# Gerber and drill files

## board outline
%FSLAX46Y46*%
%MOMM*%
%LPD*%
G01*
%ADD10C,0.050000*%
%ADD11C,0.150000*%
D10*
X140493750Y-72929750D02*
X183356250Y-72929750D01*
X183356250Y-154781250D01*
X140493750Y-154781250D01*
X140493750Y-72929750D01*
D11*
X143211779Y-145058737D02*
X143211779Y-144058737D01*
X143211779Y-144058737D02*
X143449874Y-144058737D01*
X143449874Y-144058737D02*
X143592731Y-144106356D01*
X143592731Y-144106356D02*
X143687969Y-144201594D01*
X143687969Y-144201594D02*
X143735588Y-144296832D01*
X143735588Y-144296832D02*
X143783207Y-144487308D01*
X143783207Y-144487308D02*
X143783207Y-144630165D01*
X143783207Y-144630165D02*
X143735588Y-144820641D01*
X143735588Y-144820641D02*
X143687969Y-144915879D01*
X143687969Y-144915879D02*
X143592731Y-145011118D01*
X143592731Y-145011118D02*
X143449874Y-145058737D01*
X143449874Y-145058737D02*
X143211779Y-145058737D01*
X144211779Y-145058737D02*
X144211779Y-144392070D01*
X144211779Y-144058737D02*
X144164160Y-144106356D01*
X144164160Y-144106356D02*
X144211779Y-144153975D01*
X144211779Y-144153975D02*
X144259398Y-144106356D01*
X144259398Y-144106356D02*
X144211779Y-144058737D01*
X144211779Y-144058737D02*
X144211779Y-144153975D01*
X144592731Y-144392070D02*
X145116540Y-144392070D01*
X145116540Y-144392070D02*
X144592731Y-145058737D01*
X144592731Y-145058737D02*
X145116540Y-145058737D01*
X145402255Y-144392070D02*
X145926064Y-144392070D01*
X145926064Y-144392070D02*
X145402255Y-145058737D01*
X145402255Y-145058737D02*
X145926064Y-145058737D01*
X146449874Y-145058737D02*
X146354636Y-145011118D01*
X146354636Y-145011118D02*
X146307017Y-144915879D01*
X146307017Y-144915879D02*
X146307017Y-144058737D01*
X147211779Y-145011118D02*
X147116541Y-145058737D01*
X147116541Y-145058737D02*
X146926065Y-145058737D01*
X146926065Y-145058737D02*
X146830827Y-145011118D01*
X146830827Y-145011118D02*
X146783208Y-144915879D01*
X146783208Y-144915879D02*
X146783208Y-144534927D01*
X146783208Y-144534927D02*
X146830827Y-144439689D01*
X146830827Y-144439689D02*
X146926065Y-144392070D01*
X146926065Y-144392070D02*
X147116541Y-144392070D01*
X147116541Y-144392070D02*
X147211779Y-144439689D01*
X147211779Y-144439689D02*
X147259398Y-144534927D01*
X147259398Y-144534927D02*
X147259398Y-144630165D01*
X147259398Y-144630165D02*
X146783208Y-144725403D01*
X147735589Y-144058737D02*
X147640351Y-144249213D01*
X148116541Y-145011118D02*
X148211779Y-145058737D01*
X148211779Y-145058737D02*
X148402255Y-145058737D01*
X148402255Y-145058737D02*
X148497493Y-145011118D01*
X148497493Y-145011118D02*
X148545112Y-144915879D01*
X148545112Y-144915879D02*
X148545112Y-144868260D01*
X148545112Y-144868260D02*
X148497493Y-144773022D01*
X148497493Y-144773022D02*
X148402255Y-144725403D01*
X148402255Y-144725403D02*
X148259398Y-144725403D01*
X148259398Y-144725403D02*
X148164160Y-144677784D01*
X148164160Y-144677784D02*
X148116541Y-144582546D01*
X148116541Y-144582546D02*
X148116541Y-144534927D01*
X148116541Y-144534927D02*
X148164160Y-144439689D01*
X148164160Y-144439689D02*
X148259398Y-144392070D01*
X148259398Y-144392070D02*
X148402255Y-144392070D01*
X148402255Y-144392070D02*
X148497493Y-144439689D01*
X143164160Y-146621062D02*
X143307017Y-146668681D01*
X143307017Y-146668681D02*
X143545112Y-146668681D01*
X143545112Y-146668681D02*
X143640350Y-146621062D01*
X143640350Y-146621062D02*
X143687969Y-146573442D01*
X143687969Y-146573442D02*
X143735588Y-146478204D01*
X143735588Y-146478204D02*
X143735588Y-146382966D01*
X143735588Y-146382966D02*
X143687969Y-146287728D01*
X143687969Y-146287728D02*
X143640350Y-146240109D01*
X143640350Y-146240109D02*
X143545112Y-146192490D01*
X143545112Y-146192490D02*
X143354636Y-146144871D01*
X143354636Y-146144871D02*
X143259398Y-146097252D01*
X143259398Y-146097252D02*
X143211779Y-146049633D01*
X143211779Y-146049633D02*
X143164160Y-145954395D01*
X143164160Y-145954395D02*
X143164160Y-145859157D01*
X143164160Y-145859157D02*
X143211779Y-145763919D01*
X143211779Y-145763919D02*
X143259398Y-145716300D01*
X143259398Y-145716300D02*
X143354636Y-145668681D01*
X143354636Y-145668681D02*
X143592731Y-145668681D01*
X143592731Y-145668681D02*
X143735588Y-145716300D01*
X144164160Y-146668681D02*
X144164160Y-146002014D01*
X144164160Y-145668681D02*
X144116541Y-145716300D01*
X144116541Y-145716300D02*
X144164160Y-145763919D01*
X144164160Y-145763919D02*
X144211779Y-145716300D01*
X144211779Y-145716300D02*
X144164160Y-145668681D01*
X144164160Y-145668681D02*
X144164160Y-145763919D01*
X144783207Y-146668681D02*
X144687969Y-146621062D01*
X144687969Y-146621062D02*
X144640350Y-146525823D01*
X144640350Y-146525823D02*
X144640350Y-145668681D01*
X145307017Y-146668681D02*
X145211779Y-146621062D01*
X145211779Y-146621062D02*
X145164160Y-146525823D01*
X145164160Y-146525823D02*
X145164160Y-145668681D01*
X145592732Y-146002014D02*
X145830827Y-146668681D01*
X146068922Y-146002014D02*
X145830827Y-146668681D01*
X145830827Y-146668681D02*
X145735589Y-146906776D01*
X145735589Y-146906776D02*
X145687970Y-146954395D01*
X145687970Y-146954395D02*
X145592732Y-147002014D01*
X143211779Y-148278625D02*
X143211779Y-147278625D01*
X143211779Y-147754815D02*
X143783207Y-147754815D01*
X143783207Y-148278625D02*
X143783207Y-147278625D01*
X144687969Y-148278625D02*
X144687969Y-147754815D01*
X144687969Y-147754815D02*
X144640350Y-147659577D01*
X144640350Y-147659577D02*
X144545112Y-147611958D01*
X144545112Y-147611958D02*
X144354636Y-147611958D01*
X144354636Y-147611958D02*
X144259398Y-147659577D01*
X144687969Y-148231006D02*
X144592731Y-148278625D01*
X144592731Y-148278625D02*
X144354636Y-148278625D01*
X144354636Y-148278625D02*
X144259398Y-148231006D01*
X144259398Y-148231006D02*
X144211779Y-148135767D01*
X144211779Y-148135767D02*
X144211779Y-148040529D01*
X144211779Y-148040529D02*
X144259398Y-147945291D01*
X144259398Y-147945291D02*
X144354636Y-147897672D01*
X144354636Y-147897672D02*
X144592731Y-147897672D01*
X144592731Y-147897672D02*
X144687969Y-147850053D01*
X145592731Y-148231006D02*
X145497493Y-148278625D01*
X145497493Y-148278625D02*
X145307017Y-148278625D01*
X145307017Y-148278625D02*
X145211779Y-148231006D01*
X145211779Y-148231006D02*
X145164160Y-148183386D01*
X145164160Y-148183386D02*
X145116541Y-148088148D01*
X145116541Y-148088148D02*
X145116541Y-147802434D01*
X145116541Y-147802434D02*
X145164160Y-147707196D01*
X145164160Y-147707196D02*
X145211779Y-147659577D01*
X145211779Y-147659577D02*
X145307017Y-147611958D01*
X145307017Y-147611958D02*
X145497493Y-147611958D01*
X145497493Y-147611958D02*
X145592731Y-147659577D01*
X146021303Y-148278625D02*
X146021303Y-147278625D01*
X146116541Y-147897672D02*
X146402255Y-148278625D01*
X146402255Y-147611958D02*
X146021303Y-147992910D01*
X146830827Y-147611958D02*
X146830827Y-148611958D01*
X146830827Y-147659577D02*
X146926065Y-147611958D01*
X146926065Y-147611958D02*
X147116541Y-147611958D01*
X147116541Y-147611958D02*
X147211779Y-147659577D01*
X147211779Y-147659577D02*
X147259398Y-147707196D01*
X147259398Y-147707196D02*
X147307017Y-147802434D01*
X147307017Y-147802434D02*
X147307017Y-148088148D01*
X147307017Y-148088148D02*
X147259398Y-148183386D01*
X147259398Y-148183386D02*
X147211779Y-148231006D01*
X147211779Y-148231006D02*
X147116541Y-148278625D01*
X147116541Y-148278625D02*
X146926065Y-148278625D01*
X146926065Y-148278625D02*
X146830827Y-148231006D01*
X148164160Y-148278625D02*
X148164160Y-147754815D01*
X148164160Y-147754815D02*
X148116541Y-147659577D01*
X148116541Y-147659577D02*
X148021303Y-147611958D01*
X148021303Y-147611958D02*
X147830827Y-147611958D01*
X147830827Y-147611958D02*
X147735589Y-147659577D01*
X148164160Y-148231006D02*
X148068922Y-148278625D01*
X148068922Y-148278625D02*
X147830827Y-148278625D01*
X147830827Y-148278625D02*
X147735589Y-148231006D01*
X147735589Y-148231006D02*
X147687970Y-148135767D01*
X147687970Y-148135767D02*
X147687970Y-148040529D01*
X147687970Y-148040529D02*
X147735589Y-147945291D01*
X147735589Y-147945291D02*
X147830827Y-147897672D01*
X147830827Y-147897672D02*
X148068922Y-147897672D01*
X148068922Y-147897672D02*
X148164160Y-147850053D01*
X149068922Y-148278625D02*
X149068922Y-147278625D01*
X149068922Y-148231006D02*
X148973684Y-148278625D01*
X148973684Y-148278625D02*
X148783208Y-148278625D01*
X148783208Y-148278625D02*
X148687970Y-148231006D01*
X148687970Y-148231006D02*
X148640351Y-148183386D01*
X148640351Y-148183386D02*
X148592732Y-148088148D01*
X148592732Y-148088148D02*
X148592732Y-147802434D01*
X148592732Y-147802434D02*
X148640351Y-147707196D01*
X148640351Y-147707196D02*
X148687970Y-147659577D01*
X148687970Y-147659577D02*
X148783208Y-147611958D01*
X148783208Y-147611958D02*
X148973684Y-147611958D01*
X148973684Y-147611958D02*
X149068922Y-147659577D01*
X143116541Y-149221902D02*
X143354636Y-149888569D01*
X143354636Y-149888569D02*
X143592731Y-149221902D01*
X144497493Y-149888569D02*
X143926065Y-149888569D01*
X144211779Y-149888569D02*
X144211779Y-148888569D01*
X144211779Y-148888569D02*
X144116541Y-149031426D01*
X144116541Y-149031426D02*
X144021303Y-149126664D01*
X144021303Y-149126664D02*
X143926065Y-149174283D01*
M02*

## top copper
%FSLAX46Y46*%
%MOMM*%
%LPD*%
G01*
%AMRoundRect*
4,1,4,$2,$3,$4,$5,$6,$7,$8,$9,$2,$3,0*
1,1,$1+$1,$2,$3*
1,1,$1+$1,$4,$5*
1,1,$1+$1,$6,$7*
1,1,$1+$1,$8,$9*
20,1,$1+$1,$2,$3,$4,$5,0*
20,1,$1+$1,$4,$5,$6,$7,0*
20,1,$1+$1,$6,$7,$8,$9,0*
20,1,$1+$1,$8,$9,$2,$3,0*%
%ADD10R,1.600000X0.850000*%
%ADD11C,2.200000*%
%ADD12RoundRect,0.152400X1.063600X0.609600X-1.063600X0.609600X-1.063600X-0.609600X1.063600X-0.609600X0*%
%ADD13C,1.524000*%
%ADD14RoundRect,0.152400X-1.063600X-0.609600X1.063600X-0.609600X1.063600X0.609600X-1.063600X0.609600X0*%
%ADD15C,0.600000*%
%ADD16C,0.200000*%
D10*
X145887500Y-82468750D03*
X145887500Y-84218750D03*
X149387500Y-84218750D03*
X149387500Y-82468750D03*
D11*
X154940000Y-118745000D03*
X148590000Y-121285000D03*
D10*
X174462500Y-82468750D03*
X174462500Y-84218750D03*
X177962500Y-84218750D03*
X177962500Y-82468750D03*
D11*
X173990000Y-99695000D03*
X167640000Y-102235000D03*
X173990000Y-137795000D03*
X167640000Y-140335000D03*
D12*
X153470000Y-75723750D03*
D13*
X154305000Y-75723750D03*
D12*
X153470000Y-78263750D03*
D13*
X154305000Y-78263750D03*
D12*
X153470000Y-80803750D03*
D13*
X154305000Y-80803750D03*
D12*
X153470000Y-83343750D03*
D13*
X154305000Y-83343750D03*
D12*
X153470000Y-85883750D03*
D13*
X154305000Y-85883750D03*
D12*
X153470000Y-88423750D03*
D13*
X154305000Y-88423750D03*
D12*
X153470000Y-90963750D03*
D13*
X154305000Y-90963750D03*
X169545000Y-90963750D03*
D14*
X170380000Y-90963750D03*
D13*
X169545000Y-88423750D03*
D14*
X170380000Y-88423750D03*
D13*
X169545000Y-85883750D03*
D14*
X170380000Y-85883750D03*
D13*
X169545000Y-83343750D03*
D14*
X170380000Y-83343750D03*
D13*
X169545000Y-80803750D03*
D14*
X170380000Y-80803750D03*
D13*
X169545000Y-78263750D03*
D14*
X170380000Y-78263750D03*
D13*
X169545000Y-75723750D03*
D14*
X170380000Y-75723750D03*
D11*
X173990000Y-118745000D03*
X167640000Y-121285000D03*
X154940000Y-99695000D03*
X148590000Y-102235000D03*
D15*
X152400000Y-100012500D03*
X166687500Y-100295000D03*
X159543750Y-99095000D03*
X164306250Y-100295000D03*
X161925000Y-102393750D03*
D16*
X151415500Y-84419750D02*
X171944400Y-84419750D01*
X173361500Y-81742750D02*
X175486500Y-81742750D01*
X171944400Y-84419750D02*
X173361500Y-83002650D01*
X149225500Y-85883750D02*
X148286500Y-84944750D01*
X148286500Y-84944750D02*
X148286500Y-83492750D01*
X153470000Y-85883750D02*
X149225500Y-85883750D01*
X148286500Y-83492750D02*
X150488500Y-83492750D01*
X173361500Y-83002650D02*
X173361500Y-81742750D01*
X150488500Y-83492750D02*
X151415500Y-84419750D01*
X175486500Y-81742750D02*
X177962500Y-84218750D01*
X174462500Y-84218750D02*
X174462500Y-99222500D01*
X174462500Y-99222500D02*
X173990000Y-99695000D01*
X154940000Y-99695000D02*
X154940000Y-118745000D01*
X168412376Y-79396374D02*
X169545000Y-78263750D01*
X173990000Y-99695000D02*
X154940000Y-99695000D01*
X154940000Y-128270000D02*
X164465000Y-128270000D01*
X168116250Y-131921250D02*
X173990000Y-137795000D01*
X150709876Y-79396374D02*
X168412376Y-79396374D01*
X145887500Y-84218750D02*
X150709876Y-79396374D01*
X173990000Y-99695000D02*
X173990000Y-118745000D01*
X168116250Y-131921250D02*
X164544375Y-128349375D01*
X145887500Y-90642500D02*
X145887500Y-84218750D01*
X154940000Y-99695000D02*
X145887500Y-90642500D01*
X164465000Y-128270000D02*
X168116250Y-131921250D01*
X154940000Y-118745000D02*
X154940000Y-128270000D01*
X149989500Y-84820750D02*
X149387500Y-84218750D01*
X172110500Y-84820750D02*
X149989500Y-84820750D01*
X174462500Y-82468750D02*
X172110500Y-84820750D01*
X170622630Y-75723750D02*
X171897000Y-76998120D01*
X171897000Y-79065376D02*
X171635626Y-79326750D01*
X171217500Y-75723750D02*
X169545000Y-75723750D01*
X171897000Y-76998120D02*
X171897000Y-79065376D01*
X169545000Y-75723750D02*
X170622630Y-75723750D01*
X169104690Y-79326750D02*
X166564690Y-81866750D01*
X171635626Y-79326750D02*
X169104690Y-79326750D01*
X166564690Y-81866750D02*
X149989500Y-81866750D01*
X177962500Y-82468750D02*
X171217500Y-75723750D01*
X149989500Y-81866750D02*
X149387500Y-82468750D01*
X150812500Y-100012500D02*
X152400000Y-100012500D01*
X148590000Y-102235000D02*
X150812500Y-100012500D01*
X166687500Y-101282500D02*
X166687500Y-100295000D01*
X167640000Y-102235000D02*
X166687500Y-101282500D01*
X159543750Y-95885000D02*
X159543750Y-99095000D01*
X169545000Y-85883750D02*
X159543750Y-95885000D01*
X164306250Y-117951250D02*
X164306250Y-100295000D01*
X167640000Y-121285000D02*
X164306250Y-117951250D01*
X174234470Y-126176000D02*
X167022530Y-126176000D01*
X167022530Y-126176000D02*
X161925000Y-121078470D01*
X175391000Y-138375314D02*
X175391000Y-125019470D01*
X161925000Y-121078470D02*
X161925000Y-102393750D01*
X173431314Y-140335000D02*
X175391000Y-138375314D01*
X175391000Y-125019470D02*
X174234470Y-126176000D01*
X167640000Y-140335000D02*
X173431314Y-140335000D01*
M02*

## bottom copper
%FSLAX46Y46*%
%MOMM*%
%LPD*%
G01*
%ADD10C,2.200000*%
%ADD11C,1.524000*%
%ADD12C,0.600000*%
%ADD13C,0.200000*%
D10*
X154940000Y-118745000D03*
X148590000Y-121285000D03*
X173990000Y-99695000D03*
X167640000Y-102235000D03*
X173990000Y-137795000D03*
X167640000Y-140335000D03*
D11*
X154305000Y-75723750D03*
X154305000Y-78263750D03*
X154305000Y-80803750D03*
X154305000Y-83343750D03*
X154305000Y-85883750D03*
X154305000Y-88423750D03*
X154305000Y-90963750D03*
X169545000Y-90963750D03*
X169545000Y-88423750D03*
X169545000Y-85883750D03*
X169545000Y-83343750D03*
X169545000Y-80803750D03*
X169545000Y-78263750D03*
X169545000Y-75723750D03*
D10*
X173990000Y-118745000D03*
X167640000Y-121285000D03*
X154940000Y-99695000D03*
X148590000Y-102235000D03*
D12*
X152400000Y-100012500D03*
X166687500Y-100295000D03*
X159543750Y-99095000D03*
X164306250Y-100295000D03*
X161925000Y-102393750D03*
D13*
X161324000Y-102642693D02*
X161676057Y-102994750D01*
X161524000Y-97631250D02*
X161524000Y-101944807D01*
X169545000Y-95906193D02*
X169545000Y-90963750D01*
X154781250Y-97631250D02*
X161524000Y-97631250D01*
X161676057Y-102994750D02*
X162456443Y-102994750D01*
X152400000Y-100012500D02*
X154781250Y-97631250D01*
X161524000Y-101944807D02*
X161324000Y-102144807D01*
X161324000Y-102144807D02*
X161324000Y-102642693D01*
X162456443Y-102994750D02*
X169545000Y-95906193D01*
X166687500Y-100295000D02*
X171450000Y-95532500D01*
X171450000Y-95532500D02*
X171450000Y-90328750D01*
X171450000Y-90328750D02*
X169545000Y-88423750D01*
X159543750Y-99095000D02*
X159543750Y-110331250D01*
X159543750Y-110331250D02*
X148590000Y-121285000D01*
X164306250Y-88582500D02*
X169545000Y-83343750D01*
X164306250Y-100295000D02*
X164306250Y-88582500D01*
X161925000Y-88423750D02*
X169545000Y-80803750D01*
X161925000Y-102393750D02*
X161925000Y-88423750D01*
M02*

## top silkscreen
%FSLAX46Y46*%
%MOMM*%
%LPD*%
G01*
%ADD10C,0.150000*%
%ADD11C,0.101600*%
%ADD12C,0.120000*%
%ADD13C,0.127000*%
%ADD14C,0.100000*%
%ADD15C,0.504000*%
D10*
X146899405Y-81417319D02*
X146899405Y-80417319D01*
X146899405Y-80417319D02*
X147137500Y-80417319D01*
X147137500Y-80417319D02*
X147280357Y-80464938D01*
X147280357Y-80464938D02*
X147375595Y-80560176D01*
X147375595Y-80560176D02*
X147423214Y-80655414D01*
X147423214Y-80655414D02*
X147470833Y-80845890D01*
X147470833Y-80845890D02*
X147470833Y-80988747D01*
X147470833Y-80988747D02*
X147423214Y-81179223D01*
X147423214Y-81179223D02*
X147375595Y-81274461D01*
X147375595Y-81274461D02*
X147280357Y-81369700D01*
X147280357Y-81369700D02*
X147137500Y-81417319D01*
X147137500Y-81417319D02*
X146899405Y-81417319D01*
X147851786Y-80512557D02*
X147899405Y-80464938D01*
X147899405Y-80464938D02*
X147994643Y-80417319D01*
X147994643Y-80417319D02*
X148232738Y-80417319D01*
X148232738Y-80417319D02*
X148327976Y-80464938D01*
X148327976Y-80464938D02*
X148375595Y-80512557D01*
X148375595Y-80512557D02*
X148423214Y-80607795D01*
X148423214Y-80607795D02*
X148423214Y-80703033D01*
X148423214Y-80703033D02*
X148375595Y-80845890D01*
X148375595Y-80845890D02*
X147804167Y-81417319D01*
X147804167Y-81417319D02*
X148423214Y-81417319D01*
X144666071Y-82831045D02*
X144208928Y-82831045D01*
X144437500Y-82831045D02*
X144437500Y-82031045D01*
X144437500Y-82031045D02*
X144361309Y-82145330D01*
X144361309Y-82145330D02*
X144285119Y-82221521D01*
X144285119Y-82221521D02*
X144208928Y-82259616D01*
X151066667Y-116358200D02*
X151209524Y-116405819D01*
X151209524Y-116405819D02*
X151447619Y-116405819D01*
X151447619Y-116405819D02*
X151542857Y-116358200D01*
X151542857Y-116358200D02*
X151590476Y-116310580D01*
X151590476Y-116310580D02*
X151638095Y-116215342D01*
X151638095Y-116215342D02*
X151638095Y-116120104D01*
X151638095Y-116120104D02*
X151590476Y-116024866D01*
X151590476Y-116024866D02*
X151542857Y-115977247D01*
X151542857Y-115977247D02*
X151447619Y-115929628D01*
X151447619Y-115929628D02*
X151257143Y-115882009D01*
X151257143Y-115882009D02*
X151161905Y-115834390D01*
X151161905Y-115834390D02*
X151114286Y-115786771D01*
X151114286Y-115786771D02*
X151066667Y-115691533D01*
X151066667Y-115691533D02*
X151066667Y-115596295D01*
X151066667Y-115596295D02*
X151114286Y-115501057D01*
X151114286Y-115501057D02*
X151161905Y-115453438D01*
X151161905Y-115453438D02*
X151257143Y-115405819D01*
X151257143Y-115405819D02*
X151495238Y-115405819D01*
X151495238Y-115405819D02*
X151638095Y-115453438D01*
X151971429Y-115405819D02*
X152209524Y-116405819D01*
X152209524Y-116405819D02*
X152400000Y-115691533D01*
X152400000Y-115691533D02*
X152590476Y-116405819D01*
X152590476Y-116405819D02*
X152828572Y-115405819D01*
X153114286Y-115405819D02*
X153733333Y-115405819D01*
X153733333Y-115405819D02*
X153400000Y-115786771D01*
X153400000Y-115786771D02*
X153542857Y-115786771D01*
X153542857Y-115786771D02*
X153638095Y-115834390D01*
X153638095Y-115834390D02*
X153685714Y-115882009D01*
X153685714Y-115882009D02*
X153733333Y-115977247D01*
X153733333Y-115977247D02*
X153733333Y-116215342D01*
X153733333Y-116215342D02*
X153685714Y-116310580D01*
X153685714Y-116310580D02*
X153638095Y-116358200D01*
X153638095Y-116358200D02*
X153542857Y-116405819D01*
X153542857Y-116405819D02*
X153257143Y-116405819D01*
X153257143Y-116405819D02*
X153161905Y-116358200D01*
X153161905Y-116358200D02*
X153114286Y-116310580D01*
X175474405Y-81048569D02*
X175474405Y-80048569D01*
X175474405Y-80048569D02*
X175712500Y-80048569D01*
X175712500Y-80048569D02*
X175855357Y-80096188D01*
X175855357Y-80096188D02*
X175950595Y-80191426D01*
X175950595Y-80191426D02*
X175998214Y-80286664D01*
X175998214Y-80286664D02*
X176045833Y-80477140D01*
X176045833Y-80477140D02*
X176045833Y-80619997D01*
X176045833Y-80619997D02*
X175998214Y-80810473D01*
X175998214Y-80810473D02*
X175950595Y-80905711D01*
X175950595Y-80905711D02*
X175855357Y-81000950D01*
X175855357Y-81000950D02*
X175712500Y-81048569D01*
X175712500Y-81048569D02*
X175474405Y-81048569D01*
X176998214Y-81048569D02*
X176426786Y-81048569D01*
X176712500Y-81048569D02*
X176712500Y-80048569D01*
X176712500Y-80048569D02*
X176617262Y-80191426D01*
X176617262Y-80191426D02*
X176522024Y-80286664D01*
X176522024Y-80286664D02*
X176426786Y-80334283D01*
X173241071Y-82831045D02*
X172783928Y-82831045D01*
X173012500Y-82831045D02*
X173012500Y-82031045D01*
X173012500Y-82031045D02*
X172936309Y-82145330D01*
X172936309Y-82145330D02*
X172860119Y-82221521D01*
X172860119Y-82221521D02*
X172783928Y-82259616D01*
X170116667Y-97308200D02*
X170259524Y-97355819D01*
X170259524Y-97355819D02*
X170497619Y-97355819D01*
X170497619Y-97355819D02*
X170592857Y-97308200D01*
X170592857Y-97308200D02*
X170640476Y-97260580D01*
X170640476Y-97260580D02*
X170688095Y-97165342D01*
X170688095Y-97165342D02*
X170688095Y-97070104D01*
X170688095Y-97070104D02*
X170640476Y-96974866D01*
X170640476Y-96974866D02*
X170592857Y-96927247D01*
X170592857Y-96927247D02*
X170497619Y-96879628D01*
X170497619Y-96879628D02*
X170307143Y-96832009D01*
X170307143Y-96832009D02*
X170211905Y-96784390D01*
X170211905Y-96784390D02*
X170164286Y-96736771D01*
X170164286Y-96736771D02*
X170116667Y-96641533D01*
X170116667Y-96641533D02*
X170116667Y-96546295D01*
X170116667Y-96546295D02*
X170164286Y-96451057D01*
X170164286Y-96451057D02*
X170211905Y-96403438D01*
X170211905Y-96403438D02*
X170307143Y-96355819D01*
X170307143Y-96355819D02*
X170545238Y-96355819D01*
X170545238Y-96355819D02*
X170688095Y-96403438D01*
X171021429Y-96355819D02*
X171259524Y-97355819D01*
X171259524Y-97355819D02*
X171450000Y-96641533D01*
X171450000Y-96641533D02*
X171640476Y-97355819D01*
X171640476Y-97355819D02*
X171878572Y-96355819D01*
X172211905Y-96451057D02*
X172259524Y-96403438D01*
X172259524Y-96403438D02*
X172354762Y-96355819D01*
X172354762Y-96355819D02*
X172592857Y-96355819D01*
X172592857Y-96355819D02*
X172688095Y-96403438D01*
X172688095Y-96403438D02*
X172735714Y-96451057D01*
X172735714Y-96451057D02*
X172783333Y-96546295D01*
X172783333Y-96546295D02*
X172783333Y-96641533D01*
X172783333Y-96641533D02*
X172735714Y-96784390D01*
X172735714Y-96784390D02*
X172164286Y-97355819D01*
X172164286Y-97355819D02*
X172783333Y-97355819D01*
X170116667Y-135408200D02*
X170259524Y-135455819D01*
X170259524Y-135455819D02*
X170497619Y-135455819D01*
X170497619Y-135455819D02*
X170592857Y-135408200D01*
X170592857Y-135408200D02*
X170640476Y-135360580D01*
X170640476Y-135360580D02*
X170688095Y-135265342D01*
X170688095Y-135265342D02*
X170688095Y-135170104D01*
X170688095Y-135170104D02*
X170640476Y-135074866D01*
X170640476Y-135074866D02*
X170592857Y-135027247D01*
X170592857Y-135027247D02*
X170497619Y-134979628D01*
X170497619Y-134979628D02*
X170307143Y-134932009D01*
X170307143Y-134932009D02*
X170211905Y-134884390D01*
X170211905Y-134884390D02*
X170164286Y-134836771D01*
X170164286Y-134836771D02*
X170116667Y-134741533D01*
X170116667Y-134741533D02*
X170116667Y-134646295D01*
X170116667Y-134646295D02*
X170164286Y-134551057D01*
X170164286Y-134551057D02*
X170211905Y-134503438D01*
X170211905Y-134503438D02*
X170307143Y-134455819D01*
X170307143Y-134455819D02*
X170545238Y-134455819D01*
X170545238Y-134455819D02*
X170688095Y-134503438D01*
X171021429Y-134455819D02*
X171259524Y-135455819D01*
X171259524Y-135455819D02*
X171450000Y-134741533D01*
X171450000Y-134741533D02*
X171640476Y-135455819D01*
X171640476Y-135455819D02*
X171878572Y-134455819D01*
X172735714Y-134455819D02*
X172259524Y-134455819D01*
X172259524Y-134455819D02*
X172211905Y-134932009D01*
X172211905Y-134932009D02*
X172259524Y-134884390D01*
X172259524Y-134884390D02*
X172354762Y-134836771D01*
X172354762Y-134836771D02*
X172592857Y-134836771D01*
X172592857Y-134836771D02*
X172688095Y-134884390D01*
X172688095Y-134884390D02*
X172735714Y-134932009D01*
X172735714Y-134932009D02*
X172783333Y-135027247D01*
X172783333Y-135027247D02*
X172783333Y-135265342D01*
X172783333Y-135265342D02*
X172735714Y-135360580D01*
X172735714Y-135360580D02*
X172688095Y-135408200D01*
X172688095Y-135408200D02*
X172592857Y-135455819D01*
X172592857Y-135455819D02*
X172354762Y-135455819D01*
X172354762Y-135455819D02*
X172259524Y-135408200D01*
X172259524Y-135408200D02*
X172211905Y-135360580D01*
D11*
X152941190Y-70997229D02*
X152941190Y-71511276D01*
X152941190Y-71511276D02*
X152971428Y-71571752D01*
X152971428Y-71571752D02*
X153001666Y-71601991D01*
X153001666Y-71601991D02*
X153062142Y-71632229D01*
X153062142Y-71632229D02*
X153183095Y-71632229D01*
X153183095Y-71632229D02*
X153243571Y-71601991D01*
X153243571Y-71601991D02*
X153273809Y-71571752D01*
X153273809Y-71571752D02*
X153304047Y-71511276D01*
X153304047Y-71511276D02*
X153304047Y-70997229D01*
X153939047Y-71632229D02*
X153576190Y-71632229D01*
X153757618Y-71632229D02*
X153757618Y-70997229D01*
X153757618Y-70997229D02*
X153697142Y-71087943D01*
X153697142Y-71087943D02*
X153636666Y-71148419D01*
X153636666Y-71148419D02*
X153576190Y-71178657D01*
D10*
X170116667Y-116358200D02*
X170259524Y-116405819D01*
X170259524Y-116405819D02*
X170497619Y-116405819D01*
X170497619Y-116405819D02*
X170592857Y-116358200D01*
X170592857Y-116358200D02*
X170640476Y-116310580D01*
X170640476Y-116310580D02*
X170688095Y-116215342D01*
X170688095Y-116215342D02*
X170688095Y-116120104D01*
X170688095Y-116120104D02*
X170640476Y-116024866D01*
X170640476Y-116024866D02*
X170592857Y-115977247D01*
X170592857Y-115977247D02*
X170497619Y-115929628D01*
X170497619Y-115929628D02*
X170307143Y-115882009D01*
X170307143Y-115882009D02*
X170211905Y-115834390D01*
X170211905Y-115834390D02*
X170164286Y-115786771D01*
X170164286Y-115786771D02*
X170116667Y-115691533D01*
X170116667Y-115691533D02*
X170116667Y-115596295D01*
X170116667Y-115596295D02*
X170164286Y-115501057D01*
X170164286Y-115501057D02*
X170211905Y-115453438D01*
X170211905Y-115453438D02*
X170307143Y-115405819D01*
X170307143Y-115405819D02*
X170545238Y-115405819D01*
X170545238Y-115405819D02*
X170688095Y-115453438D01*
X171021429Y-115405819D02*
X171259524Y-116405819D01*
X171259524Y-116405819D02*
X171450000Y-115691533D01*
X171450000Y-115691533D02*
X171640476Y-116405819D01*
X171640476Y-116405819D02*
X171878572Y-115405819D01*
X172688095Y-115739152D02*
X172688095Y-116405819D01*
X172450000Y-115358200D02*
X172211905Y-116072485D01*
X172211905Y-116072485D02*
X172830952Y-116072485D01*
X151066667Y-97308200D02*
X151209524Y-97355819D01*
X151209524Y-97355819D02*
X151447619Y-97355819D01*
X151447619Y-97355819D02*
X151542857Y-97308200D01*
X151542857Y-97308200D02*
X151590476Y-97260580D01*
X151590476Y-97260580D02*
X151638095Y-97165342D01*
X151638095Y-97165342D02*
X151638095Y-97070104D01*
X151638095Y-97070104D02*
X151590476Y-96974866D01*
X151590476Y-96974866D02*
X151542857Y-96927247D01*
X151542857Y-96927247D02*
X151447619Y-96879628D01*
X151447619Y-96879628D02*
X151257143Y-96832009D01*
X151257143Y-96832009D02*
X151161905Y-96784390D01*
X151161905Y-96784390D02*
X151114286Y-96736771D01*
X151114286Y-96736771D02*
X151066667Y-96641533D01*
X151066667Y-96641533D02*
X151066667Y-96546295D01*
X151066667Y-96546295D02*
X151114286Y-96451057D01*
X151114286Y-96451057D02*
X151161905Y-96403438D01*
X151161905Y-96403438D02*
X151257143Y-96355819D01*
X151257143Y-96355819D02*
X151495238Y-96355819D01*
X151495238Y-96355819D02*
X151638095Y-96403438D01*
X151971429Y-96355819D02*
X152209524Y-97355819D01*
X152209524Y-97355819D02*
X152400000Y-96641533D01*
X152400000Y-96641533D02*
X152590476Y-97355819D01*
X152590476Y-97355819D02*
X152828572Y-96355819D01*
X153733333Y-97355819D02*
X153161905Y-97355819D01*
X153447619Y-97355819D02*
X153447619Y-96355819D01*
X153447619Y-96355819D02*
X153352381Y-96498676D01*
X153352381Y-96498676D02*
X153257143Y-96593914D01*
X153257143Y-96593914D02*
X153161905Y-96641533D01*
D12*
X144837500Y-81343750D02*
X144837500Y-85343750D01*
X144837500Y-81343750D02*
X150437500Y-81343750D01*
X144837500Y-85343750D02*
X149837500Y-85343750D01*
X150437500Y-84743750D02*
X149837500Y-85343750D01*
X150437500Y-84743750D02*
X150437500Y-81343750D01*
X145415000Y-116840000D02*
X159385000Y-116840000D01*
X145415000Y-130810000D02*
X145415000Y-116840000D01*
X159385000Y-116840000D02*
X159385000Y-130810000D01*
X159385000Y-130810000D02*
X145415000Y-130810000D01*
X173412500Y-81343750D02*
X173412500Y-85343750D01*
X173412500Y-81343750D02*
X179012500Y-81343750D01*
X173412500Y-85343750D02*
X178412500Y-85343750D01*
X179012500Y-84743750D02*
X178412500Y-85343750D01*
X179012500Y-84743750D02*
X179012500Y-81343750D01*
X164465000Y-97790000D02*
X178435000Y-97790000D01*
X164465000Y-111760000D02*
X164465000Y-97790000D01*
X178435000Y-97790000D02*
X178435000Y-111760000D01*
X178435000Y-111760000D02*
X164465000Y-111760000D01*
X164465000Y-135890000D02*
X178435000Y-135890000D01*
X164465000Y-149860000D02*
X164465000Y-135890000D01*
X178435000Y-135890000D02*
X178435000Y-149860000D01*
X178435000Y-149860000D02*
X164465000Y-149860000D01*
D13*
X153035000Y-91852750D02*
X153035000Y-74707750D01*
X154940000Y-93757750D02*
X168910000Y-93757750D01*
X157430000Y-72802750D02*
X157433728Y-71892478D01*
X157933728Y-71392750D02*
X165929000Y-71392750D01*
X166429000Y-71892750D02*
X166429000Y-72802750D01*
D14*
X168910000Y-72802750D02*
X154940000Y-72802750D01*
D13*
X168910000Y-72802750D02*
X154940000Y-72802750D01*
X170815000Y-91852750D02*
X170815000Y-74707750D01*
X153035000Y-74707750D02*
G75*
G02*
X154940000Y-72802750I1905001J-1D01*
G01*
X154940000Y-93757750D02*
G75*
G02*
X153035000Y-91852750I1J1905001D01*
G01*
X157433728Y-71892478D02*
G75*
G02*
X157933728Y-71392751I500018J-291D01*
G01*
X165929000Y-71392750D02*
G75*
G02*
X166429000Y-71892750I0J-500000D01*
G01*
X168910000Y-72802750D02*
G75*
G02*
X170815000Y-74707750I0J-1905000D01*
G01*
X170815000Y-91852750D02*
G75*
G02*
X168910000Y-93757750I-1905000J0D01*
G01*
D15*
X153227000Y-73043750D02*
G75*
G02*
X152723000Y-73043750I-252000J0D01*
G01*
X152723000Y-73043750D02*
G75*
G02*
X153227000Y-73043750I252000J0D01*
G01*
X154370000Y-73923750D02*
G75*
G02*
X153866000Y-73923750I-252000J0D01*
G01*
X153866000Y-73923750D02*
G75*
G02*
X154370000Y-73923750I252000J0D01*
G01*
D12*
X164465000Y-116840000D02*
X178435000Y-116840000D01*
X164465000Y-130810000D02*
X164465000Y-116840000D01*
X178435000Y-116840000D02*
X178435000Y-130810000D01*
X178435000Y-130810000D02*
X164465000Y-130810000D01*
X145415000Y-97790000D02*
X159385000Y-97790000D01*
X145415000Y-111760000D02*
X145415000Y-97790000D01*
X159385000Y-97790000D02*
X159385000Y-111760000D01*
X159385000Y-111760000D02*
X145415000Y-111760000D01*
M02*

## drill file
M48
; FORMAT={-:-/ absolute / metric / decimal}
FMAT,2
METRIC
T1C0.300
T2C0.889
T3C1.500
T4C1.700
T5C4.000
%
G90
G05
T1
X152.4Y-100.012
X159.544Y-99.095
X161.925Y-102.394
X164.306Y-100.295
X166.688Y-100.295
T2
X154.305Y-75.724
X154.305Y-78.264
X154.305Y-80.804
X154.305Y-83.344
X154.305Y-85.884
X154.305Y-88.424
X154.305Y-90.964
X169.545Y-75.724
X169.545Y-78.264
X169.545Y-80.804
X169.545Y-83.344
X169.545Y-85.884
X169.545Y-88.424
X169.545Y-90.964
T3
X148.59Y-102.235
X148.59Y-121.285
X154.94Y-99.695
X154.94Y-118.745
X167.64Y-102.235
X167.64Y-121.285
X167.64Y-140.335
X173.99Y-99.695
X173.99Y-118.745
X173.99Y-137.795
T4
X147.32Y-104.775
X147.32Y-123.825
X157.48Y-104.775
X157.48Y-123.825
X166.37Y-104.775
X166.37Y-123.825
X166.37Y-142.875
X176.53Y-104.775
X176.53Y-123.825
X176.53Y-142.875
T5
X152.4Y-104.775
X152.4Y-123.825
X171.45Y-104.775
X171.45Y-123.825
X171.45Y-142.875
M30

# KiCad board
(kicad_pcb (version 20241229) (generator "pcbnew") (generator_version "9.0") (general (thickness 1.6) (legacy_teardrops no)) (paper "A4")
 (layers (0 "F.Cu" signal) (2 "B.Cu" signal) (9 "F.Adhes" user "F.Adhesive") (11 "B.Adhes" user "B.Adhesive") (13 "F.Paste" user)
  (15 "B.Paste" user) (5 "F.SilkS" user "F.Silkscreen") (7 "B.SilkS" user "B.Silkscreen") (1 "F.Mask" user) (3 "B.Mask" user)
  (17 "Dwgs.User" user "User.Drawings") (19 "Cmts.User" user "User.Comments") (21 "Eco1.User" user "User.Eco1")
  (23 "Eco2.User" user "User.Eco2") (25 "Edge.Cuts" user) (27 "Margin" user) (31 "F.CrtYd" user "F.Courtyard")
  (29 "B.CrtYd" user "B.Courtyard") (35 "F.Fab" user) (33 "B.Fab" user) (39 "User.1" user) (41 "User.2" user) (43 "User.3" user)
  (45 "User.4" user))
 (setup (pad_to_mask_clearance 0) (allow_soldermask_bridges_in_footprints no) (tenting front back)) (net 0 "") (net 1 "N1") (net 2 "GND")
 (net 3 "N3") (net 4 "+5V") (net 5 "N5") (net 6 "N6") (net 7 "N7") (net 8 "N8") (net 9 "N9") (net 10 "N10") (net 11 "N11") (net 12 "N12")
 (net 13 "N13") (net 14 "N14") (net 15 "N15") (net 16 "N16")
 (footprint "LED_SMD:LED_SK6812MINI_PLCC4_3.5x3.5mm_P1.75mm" (layer "F.Cu") (at 147.6375 83.34375)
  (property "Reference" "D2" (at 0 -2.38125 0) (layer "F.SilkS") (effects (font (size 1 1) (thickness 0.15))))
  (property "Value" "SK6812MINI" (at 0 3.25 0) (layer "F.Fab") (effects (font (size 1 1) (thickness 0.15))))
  (fp_line (start -2.8 -2) (end -2.8 2) (stroke (width 0.12) (type default)) (layer "F.SilkS"))
  (fp_line (start -2.8 -2) (end 2.8 -2) (stroke (width 0.12) (type solid)) (layer "F.SilkS"))
  (fp_line (start -2.8 2) (end 2.2 2) (stroke (width 0.12) (type solid)) (layer "F.SilkS"))
  (fp_line (start 2.8 1.4) (end 2.2 2) (stroke (width 0.12) (type default)) (layer "F.SilkS"))
  (fp_line (start 2.8 1.4) (end 2.8 -2) (stroke (width 0.12) (type solid)) (layer "F.SilkS"))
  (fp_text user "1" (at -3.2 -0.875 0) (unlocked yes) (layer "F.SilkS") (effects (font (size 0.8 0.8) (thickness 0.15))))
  (pad "1" smd rect (at -1.75 -0.875) (size 1.6 0.85) (layers "F.Cu" "F.Mask" "F.Paste") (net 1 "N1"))
  (pad "2" smd rect (at -1.75 0.875) (size 1.6 0.85) (layers "F.Cu" "F.Mask" "F.Paste") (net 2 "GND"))
  (pad "3" smd rect (at 1.75 0.875) (size 1.6 0.85) (layers "F.Cu" "F.Mask" "F.Paste") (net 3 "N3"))
  (pad "4" smd rect (at 1.75 -0.875) (size 1.6 0.85) (layers "F.Cu" "F.Mask" "F.Paste") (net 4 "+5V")))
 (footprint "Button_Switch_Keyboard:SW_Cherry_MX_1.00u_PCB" (layer "F.Cu") (at 154.94 118.745)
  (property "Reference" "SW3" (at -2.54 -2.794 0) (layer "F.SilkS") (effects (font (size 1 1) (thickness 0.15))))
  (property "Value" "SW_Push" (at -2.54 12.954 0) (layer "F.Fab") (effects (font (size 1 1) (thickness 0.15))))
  (fp_line (start -9.525 -1.905) (end 4.445 -1.905) (stroke (width 0.12) (type solid)) (layer "F.SilkS"))
  (fp_line (start -9.525 12.065) (end -9.525 -1.905) (stroke (width 0.12) (type solid)) (layer "F.SilkS"))
  (fp_line (start 4.445 -1.905) (end 4.445 12.065) (stroke (width 0.12) (type solid)) (layer "F.SilkS"))
  (fp_line (start 4.445 12.065) (end -9.525 12.065) (stroke (width 0.12) (type solid)) (layer "F.SilkS"))
  (pad "" np_thru_hole circle (at -7.62 5.08) (size 1.7 1.7) (drill 1.7) (layers "*.Cu" "*.Mask"))
  (pad "" np_thru_hole circle (at -2.54 5.08) (size 4 4) (drill 4) (layers "*.Cu" "*.Mask"))
  (pad "" np_thru_hole circle (at 2.54 5.08) (size 1.7 1.7) (drill 1.7) (layers "*.Cu" "*.Mask"))
  (pad "1" thru_hole circle (at 0 0) (size 2.2 2.2) (drill 1.5) (layers "*.Cu" "*.Mask") (remove_unused_layers no) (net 2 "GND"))
  (pad "2" thru_hole circle (at -6.35 2.54) (size 2.2 2.2) (drill 1.5) (layers "*.Cu" "*.Mask") (remove_unused_layers no) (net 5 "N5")))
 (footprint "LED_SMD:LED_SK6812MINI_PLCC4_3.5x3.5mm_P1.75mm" (layer "F.Cu") (at 176.2125 83.34375)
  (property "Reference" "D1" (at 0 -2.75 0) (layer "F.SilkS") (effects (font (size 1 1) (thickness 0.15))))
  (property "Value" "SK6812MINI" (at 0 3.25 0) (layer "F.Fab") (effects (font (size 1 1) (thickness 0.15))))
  (fp_line (start -2.8 -2) (end -2.8 2) (stroke (width 0.12) (type default)) (layer "F.SilkS"))
  (fp_line (start -2.8 -2) (end 2.8 -2) (stroke (width 0.12) (type solid)) (layer "F.SilkS"))
  (fp_line (start -2.8 2) (end 2.2 2) (stroke (width 0.12) (type solid)) (layer "F.SilkS"))
  (fp_line (start 2.8 1.4) (end 2.2 2) (stroke (width 0.12) (type default)) (layer "F.SilkS"))
  (fp_line (start 2.8 1.4) (end 2.8 -2) (stroke (width 0.12) (type solid)) (layer "F.SilkS"))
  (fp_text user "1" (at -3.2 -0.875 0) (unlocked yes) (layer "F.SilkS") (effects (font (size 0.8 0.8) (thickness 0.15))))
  (pad "1" smd rect (at -1.75 -0.875) (size 1.6 0.85) (layers "F.Cu" "F.Mask" "F.Paste") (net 3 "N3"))
  (pad "2" smd rect (at -1.75 0.875) (size 1.6 0.85) (layers "F.Cu" "F.Mask" "F.Paste") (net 2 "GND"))
  (pad "3" smd rect (at 1.75 0.875) (size 1.6 0.85) (layers "F.Cu" "F.Mask" "F.Paste") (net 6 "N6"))
  (pad "4" smd rect (at 1.75 -0.875) (size 1.6 0.85) (layers "F.Cu" "F.Mask" "F.Paste") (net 4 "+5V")))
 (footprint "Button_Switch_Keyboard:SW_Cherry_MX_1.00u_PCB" (layer "F.Cu") (at 173.99 99.695)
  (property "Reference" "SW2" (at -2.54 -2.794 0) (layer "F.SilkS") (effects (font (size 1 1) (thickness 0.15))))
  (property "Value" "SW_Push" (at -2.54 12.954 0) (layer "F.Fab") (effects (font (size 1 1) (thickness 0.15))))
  (fp_line (start -9.525 -1.905) (end 4.445 -1.905) (stroke (width 0.12) (type solid)) (layer "F.SilkS"))
  (fp_line (start -9.525 12.065) (end -9.525 -1.905) (stroke (width 0.12) (type solid)) (layer "F.SilkS"))
  (fp_line (start 4.445 -1.905) (end 4.445 12.065) (stroke (width 0.12) (type solid)) (layer "F.SilkS"))
  (fp_line (start 4.445 12.065) (end -9.525 12.065) (stroke (width 0.12) (type solid)) (layer "F.SilkS"))
  (pad "" np_thru_hole circle (at -7.62 5.08) (size 1.7 1.7) (drill 1.7) (layers "*.Cu" "*.Mask"))
  (pad "" np_thru_hole circle (at -2.54 5.08) (size 4 4) (drill 4) (layers "*.Cu" "*.Mask"))
  (pad "" np_thru_hole circle (at 2.54 5.08) (size 1.7 1.7) (drill 1.7) (layers "*.Cu" "*.Mask"))
  (pad "1" thru_hole circle (at 0 0) (size 2.2 2.2) (drill 1.5) (layers "*.Cu" "*.Mask") (remove_unused_layers no) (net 2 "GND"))
  (pad "2" thru_hole circle (at -6.35 2.54) (size 2.2 2.2) (drill 1.5) (layers "*.Cu" "*.Mask") (remove_unused_layers no) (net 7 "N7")))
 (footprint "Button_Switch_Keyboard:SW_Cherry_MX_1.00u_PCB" (layer "F.Cu") (at 173.99 137.795)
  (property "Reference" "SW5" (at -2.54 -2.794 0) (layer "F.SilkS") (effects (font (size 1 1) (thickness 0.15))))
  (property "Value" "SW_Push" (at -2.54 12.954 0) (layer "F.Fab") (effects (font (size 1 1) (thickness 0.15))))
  (fp_line (start -9.525 -1.905) (end 4.445 -1.905) (stroke (width 0.12) (type solid)) (layer "F.SilkS"))
  (fp_line (start -9.525 12.065) (end -9.525 -1.905) (stroke (width 0.12) (type solid)) (layer "F.SilkS"))
  (fp_line (start 4.445 -1.905) (end 4.445 12.065) (stroke (width 0.12) (type solid)) (layer "F.SilkS"))
  (fp_line (start 4.445 12.065) (end -9.525 12.065) (stroke (width 0.12) (type solid)) (layer "F.SilkS"))
  (pad "" np_thru_hole circle (at -7.62 5.08) (size 1.7 1.7) (drill 1.7) (layers "*.Cu" "*.Mask"))
  (pad "" np_thru_hole circle (at -2.54 5.08) (size 4 4) (drill 4) (layers "*.Cu" "*.Mask"))
  (pad "" np_thru_hole circle (at 2.54 5.08) (size 1.7 1.7) (drill 1.7) (layers "*.Cu" "*.Mask"))
  (pad "1" thru_hole circle (at 0 0) (size 2.2 2.2) (drill 1.5) (layers "*.Cu" "*.Mask") (remove_unused_layers no) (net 2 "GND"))
  (pad "2" thru_hole circle (at -6.35 2.54) (size 2.2 2.2) (drill 1.5) (layers "*.Cu" "*.Mask") (remove_unused_layers no) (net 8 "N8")))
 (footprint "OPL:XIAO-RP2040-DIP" (layer "F.Cu") (at 161.925 83.34375)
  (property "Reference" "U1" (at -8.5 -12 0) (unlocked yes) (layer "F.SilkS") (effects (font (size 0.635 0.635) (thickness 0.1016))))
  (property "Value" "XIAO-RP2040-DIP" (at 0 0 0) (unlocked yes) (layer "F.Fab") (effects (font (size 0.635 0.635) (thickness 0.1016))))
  (fp_line (start -8.89 8.509) (end -8.89 -8.636) (stroke (width 0.127) (type solid)) (layer "F.SilkS"))
  (fp_line (start -6.985 10.414) (end 6.985 10.414) (stroke (width 0.127) (type solid)) (layer "F.SilkS"))
  (fp_line (start -4.495 -10.541) (end -4.491272 -11.451272) (stroke (width 0.127) (type solid)) (layer "F.SilkS"))
  (fp_line (start -3.991272 -11.951) (end 4.004 -11.951) (stroke (width 0.127) (type solid)) (layer "F.SilkS"))
  (fp_line (start 4.504 -11.451) (end 4.504 -10.541) (stroke (width 0.127) (type solid)) (layer "F.SilkS"))
  (fp_line (start 6.985 -10.541) (end -6.985 -10.541) (stroke (width 0.1) (type solid)) (layer "F.SilkS"))
  (fp_line (start 6.985 -10.541) (end -6.985 -10.541) (stroke (width 0.127) (type solid)) (layer "F.SilkS"))
  (fp_line (start 8.89 8.509) (end 8.89 -8.636) (stroke (width 0.127) (type solid)) (layer "F.SilkS"))
  (fp_arc (start -8.89 -8.636) (mid -8.332038 -9.983038) (end -6.985 -10.541) (stroke (width 0.127) (type solid)) (layer "F.SilkS"))
  (fp_arc (start -6.985 10.414) (mid -8.332038 9.856038) (end -8.89 8.509) (stroke (width 0.127) (type solid)) (layer "F.SilkS"))
  (fp_arc (start -4.491272 -11.451272) (mid -4.344728 -11.80464) (end -3.991272 -11.951) (stroke (width 0.127) (type default))
   (layer "F.SilkS"))
  (fp_arc (start 4.004 -11.951) (mid 4.357553 -11.804553) (end 4.504 -11.451) (stroke (width 0.127) (type default)) (layer "F.SilkS"))
  (fp_arc (start 6.985 -10.541) (mid 8.332038 -9.983038) (end 8.89 -8.636) (stroke (width 0.127) (type solid)) (layer "F.SilkS"))
  (fp_arc (start 8.89 8.509) (mid 8.332038 9.856038) (end 6.985 10.414) (stroke (width 0.127) (type solid)) (layer "F.SilkS"))
  (fp_circle (center -8.95 -10.3) (end -8.95 -10.554) (stroke (width 0.5) (type solid)) (fill yes) (layer "F.SilkS"))
  (fp_circle (center -7.807 -9.42) (end -7.807 -9.674) (stroke (width 0.5) (type solid)) (fill yes) (layer "F.SilkS"))
  (pad "1" smd roundrect (at -8.455 -7.62 180) (size 2.432 1.524) (layers "F.Cu" "F.Mask") (roundrect_rratio 0.1) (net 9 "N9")
   (thermal_bridge_angle 45))
  (pad "1" thru_hole circle (at -7.62 -7.62 180) (size 1.524 1.524) (drill 0.889) (layers "*.Cu" "*.Mask") (remove_unused_layers no)
   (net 9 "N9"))
  (pad "2" smd roundrect (at -8.455 -5.08 180) (size 2.432 1.524) (layers "F.Cu" "F.Mask") (roundrect_rratio 0.1) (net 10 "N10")
   (thermal_bridge_angle 45))
  (pad "2" thru_hole circle (at -7.62 -5.08 180) (size 1.524 1.524) (drill 0.889) (layers "*.Cu" "*.Mask") (remove_unused_layers no)
   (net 10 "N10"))
  (pad "3" smd roundrect (at -8.455 -2.54 180) (size 2.432 1.524) (layers "F.Cu" "F.Mask") (roundrect_rratio 0.1) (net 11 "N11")
   (thermal_bridge_angle 45))
  (pad "3" thru_hole circle (at -7.62 -2.54 180) (size 1.524 1.524) (drill 0.889) (layers "*.Cu" "*.Mask") (remove_unused_layers no)
   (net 11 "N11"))
  (pad "4" smd roundrect (at -8.455 0 180) (size 2.432 1.524) (layers "F.Cu" "F.Mask") (roundrect_rratio 0.1) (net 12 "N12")
   (thermal_bridge_angle 45))
  (pad "4" thru_hole circle (at -7.62 0 180) (size 1.524 1.524) (drill 0.889) (layers "*.Cu" "*.Mask") (remove_unused_layers no)
   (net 12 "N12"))
  (pad "5" smd roundrect (at -8.455 2.54 180) (size 2.432 1.524) (layers "F.Cu" "F.Mask") (roundrect_rratio 0.1) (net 6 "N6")
   (thermal_bridge_angle 45))
  (pad "5" thru_hole circle (at -7.62 2.54 180) (size 1.524 1.524) (drill 0.889) (layers "*.Cu" "*.Mask") (remove_unused_layers no)
   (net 6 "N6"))
  (pad "6" smd roundrect (at -8.455 5.08 180) (size 2.432 1.524) (layers "F.Cu" "F.Mask") (roundrect_rratio 0.1) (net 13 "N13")
   (thermal_bridge_angle 45))
  (pad "6" thru_hole circle (at -7.62 5.08 180) (size 1.524 1.524) (drill 0.889) (layers "*.Cu" "*.Mask") (remove_unused_layers no)
   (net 13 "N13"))
  (pad "7" smd roundrect (at -8.455 7.62 180) (size 2.432 1.524) (layers "F.Cu" "F.Mask") (roundrect_rratio 0.1) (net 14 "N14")
   (thermal_bridge_angle 45))
  (pad "7" thru_hole circle (at -7.62 7.62 180) (size 1.524 1.524) (drill 0.889) (layers "*.Cu" "*.Mask") (remove_unused_layers no)
   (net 14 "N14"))
  (pad "8" thru_hole circle (at 7.62 7.62) (size 1.524 1.524) (drill 0.889) (layers "*.Cu" "*.Mask") (remove_unused_layers no)
   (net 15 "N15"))
  (pad "8" smd roundrect (at 8.455 7.62) (size 2.432 1.524) (layers "F.Cu" "F.Mask") (roundrect_rratio 0.1) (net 15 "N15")
   (thermal_bridge_angle 45))
  (pad "9" thru_hole circle (at 7.62 5.08) (size 1.524 1.524) (drill 0.889) (layers "*.Cu" "*.Mask") (remove_unused_layers no) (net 7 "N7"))
  (pad "9" smd roundrect (at 8.455 5.08) (size 2.432 1.524) (layers "F.Cu" "F.Mask") (roundrect_rratio 0.1) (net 7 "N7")
   (thermal_bridge_angle 45))
  (pad "10" thru_hole circle (at 7.62 2.54) (size 1.524 1.524) (drill 0.889) (layers "*.Cu" "*.Mask") (remove_unused_layers no) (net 5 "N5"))
  (pad "10" smd roundrect (at 8.455 2.54) (size 2.432 1.524) (layers "F.Cu" "F.Mask") (roundrect_rratio 0.1) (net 5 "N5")
   (thermal_bridge_angle 45))
  (pad "11" thru_hole circle (at 7.62 0) (size 1.524 1.524) (drill 0.889) (layers "*.Cu" "*.Mask") (remove_unused_layers no) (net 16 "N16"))
  (pad "11" smd roundrect (at 8.455 0) (size 2.432 1.524) (layers "F.Cu" "F.Mask") (roundrect_rratio 0.1) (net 16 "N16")
   (thermal_bridge_angle 45))
  (pad "12" thru_hole circle (at 7.62 -2.54) (size 1.524 1.524) (drill 0.889) (layers "*.Cu" "*.Mask") (remove_unused_layers no)
   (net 8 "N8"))
  (pad "12" smd roundrect (at 8.455 -2.54) (size 2.432 1.524) (layers "F.Cu" "F.Mask") (roundrect_rratio 0.1) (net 8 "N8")
   (thermal_bridge_angle 45))
  (pad "13" thru_hole circle (at 7.62 -5.08) (size 1.524 1.524) (drill 0.889) (layers "*.Cu" "*.Mask") (remove_unused_layers no)
   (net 2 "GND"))
  (pad "13" smd roundrect (at 8.455 -5.08) (size 2.432 1.524) (layers "F.Cu" "F.Mask") (roundrect_rratio 0.1) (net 2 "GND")
   (thermal_bridge_angle 45))
  (pad "14" thru_hole circle (at 7.62 -7.62) (size 1.524 1.524) (drill 0.889) (layers "*.Cu" "*.Mask") (remove_unused_layers no)
   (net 4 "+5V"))
  (pad "14" smd roundrect (at 8.455 -7.62) (size 2.432 1.524) (layers "F.Cu" "F.Mask") (roundrect_rratio 0.1) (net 4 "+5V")
   (thermal_bridge_angle 45)))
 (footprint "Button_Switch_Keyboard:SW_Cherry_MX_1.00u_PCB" (layer "F.Cu") (at 173.99 118.745)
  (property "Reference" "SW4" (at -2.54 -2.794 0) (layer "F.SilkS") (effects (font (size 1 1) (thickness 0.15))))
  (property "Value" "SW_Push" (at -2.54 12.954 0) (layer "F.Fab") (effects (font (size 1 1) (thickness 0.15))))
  (fp_line (start -9.525 -1.905) (end 4.445 -1.905) (stroke (width 0.12) (type solid)) (layer "F.SilkS"))
  (fp_line (start -9.525 12.065) (end -9.525 -1.905) (stroke (width 0.12) (type solid)) (layer "F.SilkS"))
  (fp_line (start 4.445 -1.905) (end 4.445 12.065) (stroke (width 0.12) (type solid)) (layer "F.SilkS"))
  (fp_line (start 4.445 12.065) (end -9.525 12.065) (stroke (width 0.12) (type solid)) (layer "F.SilkS"))
  (pad "" np_thru_hole circle (at -7.62 5.08) (size 1.7 1.7) (drill 1.7) (layers "*.Cu" "*.Mask"))
  (pad "" np_thru_hole circle (at -2.54 5.08) (size 4 4) (drill 4) (layers "*.Cu" "*.Mask"))
  (pad "" np_thru_hole circle (at 2.54 5.08) (size 1.7 1.7) (drill 1.7) (layers "*.Cu" "*.Mask"))
  (pad "1" thru_hole circle (at 0 0) (size 2.2 2.2) (drill 1.5) (layers "*.Cu" "*.Mask") (remove_unused_layers no) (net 2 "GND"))
  (pad "2" thru_hole circle (at -6.35 2.54) (size 2.2 2.2) (drill 1.5) (layers "*.Cu" "*.Mask") (remove_unused_layers no) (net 16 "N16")))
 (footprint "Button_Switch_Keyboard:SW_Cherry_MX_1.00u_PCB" (layer "F.Cu") (at 154.94 99.695)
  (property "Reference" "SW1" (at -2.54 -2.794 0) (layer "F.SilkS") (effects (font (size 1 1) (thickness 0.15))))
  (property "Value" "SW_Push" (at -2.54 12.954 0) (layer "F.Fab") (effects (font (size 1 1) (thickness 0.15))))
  (fp_line (start -9.525 -1.905) (end 4.445 -1.905) (stroke (width 0.12) (type solid)) (layer "F.SilkS"))
  (fp_line (start -9.525 12.065) (end -9.525 -1.905) (stroke (width 0.12) (type solid)) (layer "F.SilkS"))
  (fp_line (start 4.445 -1.905) (end 4.445 12.065) (stroke (width 0.12) (type solid)) (layer "F.SilkS"))
  (fp_line (start 4.445 12.065) (end -9.525 12.065) (stroke (width 0.12) (type solid)) (layer "F.SilkS"))
  (pad "" np_thru_hole circle (at -7.62 5.08) (size 1.7 1.7) (drill 1.7) (layers "*.Cu" "*.Mask"))
  (pad "" np_thru_hole circle (at -2.54 5.08) (size 4 4) (drill 4) (layers "*.Cu" "*.Mask"))
  (pad "" np_thru_hole circle (at 2.54 5.08) (size 1.7 1.7) (drill 1.7) (layers "*.Cu" "*.Mask"))
  (pad "1" thru_hole circle (at 0 0) (size 2.2 2.2) (drill 1.5) (layers "*.Cu" "*.Mask") (remove_unused_layers no) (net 2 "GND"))
  (pad "2" thru_hole circle (at -6.35 2.54) (size 2.2 2.2) (drill 1.5) (layers "*.Cu" "*.Mask") (remove_unused_layers no) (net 15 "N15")))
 (gr_rect (start 140.49375 72.92975) (end 183.35625 154.78125) (stroke (width 0.05) (type default)) (fill no) (layer "Edge.Cuts"))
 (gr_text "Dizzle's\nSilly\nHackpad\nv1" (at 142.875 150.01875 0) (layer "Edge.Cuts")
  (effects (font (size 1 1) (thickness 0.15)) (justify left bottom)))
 (segment (start 151.4155 84.41975) (end 171.9444 84.41975) (width 0.2) (layer "F.Cu") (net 6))
 (segment (start 173.3615 81.74275) (end 175.4865 81.74275) (width 0.2) (layer "F.Cu") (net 6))
 (segment (start 171.9444 84.41975) (end 173.3615 83.00265) (width 0.2) (layer "F.Cu") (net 6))
 (segment (start 149.2255 85.88375) (end 148.2865 84.94475) (width 0.2) (layer "F.Cu") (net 6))
 (segment (start 148.2865 84.94475) (end 148.2865 83.49275) (width 0.2) (layer "F.Cu") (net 6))
 (segment (start 153.47 85.88375) (end 149.2255 85.88375) (width 0.2) (layer "F.Cu") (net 6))
 (segment (start 148.2865 83.49275) (end 150.4885 83.49275) (width 0.2) (layer "F.Cu") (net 6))
 (segment (start 173.3615 83.00265) (end 173.3615 81.74275) (width 0.2) (layer "F.Cu") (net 6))
 (segment (start 150.4885 83.49275) (end 151.4155 84.41975) (width 0.2) (layer "F.Cu") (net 6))
 (segment (start 175.4865 81.74275) (end 177.9625 84.21875) (width 0.2) (layer "F.Cu") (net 6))
 (segment (start 174.4625 84.21875) (end 174.4625 99.2225) (width 0.2) (layer "F.Cu") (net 2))
 (segment (start 174.4625 99.2225) (end 173.99 99.695) (width 0.2) (layer "F.Cu") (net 2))
 (segment (start 154.94 99.695) (end 154.94 118.745) (width 0.2) (layer "F.Cu") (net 2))
 (segment (start 168.412376 79.396374) (end 169.545 78.26375) (width 0.2) (layer "F.Cu") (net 2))
 (segment (start 173.99 99.695) (end 154.94 99.695) (width 0.2) (layer "F.Cu") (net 2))
 (segment (start 154.94 128.27) (end 164.465 128.27) (width 0.2) (layer "F.Cu") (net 2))
 (segment (start 168.11625 131.92125) (end 173.99 137.795) (width 0.2) (layer "F.Cu") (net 2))
 (segment (start 150.709876 79.396374) (end 168.412376 79.396374) (width 0.2) (layer "F.Cu") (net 2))
 (segment (start 145.8875 84.21875) (end 150.709876 79.396374) (width 0.2) (layer "F.Cu") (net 2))
 (segment (start 173.99 99.695) (end 173.99 118.745) (width 0.2) (layer "F.Cu") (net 2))
 (segment (start 168.11625 131.92125) (end 164.544375 128.349375) (width 0.2) (layer "F.Cu") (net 2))
 (segment (start 145.8875 90.6425) (end 145.8875 84.21875) (width 0.2) (layer "F.Cu") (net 2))
 (segment (start 154.94 99.695) (end 145.8875 90.6425) (width 0.2) (layer "F.Cu") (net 2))
 (segment (start 164.465 128.27) (end 168.11625 131.92125) (width 0.2) (layer "F.Cu") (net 2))
 (segment (start 154.94 118.745) (end 154.94 128.27) (width 0.2) (layer "F.Cu") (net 2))
 (segment (start 149.9895 84.82075) (end 149.3875 84.21875) (width 0.2) (layer "F.Cu") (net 3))
 (segment (start 172.1105 84.82075) (end 149.9895 84.82075) (width 0.2) (layer "F.Cu") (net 3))
 (segment (start 174.4625 82.46875) (end 172.1105 84.82075) (width 0.2) (layer "F.Cu") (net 3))
 (segment (start 170.62263 75.72375) (end 171.897 76.99812) (width 0.2) (layer "F.Cu") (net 4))
 (segment (start 171.897 79.065376) (end 171.635626 79.32675) (width 0.2) (layer "F.Cu") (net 4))
 (segment (start 171.2175 75.72375) (end 169.545 75.72375) (width 0.2) (layer "F.Cu") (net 4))
 (segment (start 171.897 76.99812) (end 171.897 79.065376) (width 0.2) (layer "F.Cu") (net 4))
 (segment (start 169.545 75.72375) (end 170.62263 75.72375) (width 0.2) (layer "F.Cu") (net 4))
 (segment (start 169.10469 79.32675) (end 166.56469 81.86675) (width 0.2) (layer "F.Cu") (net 4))
 (segment (start 171.635626 79.32675) (end 169.10469 79.32675) (width 0.2) (layer "F.Cu") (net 4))
 (segment (start 166.56469 81.86675) (end 149.9895 81.86675) (width 0.2) (layer "F.Cu") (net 4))
 (segment (start 177.9625 82.46875) (end 171.2175 75.72375) (width 0.2) (layer "F.Cu") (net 4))
 (segment (start 149.9895 81.86675) (end 149.3875 82.46875) (width 0.2) (layer "F.Cu") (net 4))
 (segment (start 150.8125 100.0125) (end 152.4 100.0125) (width 0.2) (layer "F.Cu") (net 15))
 (segment (start 148.59 102.235) (end 150.8125 100.0125) (width 0.2) (layer "F.Cu") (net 15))
 (via (at 152.4 100.0125) (size 0.6) (drill 0.3) (layers "F.Cu" "B.Cu") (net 15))
 (segment (start 161.324 102.642693) (end 161.676057 102.99475) (width 0.2) (layer "B.Cu") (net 15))
 (segment (start 161.524 97.63125) (end 161.524 101.944807) (width 0.2) (layer "B.Cu") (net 15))
 (segment (start 169.545 95.906193) (end 169.545 90.96375) (width 0.2) (layer "B.Cu") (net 15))
 (segment (start 154.78125 97.63125) (end 161.524 97.63125) (width 0.2) (layer "B.Cu") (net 15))
 (segment (start 161.676057 102.99475) (end 162.456443 102.99475) (width 0.2) (layer "B.Cu") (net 15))
 (segment (start 152.4 100.0125) (end 154.78125 97.63125) (width 0.2) (layer "B.Cu") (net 15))
 (segment (start 161.524 101.944807) (end 161.324 102.144807) (width 0.2) (layer "B.Cu") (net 15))
 (segment (start 161.324 102.144807) (end 161.324 102.642693) (width 0.2) (layer "B.Cu") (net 15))
 (segment (start 162.456443 102.99475) (end 169.545 95.906193) (width 0.2) (layer "B.Cu") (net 15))
 (segment (start 166.6875 101.2825) (end 166.6875 100.295) (width 0.2) (layer "F.Cu") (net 7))
 (segment (start 167.64 102.235) (end 166.6875 101.2825) (width 0.2) (layer "F.Cu") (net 7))
 (via (at 166.6875 100.295) (size 0.6) (drill 0.3) (layers "F.Cu" "B.Cu") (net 7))
 (segment (start 166.6875 100.295) (end 171.45 95.5325) (width 0.2) (layer "B.Cu") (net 7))
 (segment (start 171.45 95.5325) (end 171.45 90.32875) (width 0.2) (layer "B.Cu") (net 7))
 (segment (start 171.45 90.32875) (end 169.545 88.42375) (width 0.2) (layer "B.Cu") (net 7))
 (segment (start 159.54375 95.885) (end 159.54375 99.095) (width 0.2) (layer "F.Cu") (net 5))
 (segment (start 169.545 85.88375) (end 159.54375 95.885) (width 0.2) (layer "F.Cu") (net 5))
 (via (at 159.54375 99.095) (size 0.6) (drill 0.3) (layers "F.Cu" "B.Cu") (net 5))
 (segment (start 159.54375 99.095) (end 159.54375 110.33125) (width 0.2) (layer "B.Cu") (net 5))
 (segment (start 159.54375 110.33125) (end 148.59 121.285) (width 0.2) (layer "B.Cu") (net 5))
 (segment (start 164.30625 117.95125) (end 164.30625 100.295) (width 0.2) (layer "F.Cu") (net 16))
 (segment (start 167.64 121.285) (end 164.30625 117.95125) (width 0.2) (layer "F.Cu") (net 16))
 (via (at 164.30625 100.295) (size 0.6) (drill 0.3) (layers "F.Cu" "B.Cu") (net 16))
 (segment (start 164.30625 88.5825) (end 169.545 83.34375) (width 0.2) (layer "B.Cu") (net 16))
 (segment (start 164.30625 100.295) (end 164.30625 88.5825) (width 0.2) (layer "B.Cu") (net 16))
 (segment (start 174.23447 126.176) (end 167.02253 126.176) (width 0.2) (layer "F.Cu") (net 8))
 (segment (start 167.02253 126.176) (end 161.925 121.07847) (width 0.2) (layer "F.Cu") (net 8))
 (segment (start 175.391 138.375314) (end 175.391 125.01947) (width 0.2) (layer "F.Cu") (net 8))
 (segment (start 161.925 121.07847) (end 161.925 102.39375) (width 0.2) (layer "F.Cu") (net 8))
 (segment (start 173.431314 140.335) (end 175.391 138.375314) (width 0.2) (layer "F.Cu") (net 8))
 (segment (start 175.391 125.01947) (end 174.23447 126.176) (width 0.2) (layer "F.Cu") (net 8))
 (segment (start 167.64 140.335) (end 173.431314 140.335) (width 0.2) (layer "F.Cu") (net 8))
 (via (at 161.925 102.39375) (size 0.6) (drill 0.3) (layers "F.Cu" "B.Cu") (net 8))
 (segment (start 161.925 88.42375) (end 169.545 80.80375) (width 0.2) (layer "B.Cu") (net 8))
 (segment (start 161.925 102.39375) (end 161.925 88.42375) (width 0.2) (layer "B.Cu") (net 8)))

